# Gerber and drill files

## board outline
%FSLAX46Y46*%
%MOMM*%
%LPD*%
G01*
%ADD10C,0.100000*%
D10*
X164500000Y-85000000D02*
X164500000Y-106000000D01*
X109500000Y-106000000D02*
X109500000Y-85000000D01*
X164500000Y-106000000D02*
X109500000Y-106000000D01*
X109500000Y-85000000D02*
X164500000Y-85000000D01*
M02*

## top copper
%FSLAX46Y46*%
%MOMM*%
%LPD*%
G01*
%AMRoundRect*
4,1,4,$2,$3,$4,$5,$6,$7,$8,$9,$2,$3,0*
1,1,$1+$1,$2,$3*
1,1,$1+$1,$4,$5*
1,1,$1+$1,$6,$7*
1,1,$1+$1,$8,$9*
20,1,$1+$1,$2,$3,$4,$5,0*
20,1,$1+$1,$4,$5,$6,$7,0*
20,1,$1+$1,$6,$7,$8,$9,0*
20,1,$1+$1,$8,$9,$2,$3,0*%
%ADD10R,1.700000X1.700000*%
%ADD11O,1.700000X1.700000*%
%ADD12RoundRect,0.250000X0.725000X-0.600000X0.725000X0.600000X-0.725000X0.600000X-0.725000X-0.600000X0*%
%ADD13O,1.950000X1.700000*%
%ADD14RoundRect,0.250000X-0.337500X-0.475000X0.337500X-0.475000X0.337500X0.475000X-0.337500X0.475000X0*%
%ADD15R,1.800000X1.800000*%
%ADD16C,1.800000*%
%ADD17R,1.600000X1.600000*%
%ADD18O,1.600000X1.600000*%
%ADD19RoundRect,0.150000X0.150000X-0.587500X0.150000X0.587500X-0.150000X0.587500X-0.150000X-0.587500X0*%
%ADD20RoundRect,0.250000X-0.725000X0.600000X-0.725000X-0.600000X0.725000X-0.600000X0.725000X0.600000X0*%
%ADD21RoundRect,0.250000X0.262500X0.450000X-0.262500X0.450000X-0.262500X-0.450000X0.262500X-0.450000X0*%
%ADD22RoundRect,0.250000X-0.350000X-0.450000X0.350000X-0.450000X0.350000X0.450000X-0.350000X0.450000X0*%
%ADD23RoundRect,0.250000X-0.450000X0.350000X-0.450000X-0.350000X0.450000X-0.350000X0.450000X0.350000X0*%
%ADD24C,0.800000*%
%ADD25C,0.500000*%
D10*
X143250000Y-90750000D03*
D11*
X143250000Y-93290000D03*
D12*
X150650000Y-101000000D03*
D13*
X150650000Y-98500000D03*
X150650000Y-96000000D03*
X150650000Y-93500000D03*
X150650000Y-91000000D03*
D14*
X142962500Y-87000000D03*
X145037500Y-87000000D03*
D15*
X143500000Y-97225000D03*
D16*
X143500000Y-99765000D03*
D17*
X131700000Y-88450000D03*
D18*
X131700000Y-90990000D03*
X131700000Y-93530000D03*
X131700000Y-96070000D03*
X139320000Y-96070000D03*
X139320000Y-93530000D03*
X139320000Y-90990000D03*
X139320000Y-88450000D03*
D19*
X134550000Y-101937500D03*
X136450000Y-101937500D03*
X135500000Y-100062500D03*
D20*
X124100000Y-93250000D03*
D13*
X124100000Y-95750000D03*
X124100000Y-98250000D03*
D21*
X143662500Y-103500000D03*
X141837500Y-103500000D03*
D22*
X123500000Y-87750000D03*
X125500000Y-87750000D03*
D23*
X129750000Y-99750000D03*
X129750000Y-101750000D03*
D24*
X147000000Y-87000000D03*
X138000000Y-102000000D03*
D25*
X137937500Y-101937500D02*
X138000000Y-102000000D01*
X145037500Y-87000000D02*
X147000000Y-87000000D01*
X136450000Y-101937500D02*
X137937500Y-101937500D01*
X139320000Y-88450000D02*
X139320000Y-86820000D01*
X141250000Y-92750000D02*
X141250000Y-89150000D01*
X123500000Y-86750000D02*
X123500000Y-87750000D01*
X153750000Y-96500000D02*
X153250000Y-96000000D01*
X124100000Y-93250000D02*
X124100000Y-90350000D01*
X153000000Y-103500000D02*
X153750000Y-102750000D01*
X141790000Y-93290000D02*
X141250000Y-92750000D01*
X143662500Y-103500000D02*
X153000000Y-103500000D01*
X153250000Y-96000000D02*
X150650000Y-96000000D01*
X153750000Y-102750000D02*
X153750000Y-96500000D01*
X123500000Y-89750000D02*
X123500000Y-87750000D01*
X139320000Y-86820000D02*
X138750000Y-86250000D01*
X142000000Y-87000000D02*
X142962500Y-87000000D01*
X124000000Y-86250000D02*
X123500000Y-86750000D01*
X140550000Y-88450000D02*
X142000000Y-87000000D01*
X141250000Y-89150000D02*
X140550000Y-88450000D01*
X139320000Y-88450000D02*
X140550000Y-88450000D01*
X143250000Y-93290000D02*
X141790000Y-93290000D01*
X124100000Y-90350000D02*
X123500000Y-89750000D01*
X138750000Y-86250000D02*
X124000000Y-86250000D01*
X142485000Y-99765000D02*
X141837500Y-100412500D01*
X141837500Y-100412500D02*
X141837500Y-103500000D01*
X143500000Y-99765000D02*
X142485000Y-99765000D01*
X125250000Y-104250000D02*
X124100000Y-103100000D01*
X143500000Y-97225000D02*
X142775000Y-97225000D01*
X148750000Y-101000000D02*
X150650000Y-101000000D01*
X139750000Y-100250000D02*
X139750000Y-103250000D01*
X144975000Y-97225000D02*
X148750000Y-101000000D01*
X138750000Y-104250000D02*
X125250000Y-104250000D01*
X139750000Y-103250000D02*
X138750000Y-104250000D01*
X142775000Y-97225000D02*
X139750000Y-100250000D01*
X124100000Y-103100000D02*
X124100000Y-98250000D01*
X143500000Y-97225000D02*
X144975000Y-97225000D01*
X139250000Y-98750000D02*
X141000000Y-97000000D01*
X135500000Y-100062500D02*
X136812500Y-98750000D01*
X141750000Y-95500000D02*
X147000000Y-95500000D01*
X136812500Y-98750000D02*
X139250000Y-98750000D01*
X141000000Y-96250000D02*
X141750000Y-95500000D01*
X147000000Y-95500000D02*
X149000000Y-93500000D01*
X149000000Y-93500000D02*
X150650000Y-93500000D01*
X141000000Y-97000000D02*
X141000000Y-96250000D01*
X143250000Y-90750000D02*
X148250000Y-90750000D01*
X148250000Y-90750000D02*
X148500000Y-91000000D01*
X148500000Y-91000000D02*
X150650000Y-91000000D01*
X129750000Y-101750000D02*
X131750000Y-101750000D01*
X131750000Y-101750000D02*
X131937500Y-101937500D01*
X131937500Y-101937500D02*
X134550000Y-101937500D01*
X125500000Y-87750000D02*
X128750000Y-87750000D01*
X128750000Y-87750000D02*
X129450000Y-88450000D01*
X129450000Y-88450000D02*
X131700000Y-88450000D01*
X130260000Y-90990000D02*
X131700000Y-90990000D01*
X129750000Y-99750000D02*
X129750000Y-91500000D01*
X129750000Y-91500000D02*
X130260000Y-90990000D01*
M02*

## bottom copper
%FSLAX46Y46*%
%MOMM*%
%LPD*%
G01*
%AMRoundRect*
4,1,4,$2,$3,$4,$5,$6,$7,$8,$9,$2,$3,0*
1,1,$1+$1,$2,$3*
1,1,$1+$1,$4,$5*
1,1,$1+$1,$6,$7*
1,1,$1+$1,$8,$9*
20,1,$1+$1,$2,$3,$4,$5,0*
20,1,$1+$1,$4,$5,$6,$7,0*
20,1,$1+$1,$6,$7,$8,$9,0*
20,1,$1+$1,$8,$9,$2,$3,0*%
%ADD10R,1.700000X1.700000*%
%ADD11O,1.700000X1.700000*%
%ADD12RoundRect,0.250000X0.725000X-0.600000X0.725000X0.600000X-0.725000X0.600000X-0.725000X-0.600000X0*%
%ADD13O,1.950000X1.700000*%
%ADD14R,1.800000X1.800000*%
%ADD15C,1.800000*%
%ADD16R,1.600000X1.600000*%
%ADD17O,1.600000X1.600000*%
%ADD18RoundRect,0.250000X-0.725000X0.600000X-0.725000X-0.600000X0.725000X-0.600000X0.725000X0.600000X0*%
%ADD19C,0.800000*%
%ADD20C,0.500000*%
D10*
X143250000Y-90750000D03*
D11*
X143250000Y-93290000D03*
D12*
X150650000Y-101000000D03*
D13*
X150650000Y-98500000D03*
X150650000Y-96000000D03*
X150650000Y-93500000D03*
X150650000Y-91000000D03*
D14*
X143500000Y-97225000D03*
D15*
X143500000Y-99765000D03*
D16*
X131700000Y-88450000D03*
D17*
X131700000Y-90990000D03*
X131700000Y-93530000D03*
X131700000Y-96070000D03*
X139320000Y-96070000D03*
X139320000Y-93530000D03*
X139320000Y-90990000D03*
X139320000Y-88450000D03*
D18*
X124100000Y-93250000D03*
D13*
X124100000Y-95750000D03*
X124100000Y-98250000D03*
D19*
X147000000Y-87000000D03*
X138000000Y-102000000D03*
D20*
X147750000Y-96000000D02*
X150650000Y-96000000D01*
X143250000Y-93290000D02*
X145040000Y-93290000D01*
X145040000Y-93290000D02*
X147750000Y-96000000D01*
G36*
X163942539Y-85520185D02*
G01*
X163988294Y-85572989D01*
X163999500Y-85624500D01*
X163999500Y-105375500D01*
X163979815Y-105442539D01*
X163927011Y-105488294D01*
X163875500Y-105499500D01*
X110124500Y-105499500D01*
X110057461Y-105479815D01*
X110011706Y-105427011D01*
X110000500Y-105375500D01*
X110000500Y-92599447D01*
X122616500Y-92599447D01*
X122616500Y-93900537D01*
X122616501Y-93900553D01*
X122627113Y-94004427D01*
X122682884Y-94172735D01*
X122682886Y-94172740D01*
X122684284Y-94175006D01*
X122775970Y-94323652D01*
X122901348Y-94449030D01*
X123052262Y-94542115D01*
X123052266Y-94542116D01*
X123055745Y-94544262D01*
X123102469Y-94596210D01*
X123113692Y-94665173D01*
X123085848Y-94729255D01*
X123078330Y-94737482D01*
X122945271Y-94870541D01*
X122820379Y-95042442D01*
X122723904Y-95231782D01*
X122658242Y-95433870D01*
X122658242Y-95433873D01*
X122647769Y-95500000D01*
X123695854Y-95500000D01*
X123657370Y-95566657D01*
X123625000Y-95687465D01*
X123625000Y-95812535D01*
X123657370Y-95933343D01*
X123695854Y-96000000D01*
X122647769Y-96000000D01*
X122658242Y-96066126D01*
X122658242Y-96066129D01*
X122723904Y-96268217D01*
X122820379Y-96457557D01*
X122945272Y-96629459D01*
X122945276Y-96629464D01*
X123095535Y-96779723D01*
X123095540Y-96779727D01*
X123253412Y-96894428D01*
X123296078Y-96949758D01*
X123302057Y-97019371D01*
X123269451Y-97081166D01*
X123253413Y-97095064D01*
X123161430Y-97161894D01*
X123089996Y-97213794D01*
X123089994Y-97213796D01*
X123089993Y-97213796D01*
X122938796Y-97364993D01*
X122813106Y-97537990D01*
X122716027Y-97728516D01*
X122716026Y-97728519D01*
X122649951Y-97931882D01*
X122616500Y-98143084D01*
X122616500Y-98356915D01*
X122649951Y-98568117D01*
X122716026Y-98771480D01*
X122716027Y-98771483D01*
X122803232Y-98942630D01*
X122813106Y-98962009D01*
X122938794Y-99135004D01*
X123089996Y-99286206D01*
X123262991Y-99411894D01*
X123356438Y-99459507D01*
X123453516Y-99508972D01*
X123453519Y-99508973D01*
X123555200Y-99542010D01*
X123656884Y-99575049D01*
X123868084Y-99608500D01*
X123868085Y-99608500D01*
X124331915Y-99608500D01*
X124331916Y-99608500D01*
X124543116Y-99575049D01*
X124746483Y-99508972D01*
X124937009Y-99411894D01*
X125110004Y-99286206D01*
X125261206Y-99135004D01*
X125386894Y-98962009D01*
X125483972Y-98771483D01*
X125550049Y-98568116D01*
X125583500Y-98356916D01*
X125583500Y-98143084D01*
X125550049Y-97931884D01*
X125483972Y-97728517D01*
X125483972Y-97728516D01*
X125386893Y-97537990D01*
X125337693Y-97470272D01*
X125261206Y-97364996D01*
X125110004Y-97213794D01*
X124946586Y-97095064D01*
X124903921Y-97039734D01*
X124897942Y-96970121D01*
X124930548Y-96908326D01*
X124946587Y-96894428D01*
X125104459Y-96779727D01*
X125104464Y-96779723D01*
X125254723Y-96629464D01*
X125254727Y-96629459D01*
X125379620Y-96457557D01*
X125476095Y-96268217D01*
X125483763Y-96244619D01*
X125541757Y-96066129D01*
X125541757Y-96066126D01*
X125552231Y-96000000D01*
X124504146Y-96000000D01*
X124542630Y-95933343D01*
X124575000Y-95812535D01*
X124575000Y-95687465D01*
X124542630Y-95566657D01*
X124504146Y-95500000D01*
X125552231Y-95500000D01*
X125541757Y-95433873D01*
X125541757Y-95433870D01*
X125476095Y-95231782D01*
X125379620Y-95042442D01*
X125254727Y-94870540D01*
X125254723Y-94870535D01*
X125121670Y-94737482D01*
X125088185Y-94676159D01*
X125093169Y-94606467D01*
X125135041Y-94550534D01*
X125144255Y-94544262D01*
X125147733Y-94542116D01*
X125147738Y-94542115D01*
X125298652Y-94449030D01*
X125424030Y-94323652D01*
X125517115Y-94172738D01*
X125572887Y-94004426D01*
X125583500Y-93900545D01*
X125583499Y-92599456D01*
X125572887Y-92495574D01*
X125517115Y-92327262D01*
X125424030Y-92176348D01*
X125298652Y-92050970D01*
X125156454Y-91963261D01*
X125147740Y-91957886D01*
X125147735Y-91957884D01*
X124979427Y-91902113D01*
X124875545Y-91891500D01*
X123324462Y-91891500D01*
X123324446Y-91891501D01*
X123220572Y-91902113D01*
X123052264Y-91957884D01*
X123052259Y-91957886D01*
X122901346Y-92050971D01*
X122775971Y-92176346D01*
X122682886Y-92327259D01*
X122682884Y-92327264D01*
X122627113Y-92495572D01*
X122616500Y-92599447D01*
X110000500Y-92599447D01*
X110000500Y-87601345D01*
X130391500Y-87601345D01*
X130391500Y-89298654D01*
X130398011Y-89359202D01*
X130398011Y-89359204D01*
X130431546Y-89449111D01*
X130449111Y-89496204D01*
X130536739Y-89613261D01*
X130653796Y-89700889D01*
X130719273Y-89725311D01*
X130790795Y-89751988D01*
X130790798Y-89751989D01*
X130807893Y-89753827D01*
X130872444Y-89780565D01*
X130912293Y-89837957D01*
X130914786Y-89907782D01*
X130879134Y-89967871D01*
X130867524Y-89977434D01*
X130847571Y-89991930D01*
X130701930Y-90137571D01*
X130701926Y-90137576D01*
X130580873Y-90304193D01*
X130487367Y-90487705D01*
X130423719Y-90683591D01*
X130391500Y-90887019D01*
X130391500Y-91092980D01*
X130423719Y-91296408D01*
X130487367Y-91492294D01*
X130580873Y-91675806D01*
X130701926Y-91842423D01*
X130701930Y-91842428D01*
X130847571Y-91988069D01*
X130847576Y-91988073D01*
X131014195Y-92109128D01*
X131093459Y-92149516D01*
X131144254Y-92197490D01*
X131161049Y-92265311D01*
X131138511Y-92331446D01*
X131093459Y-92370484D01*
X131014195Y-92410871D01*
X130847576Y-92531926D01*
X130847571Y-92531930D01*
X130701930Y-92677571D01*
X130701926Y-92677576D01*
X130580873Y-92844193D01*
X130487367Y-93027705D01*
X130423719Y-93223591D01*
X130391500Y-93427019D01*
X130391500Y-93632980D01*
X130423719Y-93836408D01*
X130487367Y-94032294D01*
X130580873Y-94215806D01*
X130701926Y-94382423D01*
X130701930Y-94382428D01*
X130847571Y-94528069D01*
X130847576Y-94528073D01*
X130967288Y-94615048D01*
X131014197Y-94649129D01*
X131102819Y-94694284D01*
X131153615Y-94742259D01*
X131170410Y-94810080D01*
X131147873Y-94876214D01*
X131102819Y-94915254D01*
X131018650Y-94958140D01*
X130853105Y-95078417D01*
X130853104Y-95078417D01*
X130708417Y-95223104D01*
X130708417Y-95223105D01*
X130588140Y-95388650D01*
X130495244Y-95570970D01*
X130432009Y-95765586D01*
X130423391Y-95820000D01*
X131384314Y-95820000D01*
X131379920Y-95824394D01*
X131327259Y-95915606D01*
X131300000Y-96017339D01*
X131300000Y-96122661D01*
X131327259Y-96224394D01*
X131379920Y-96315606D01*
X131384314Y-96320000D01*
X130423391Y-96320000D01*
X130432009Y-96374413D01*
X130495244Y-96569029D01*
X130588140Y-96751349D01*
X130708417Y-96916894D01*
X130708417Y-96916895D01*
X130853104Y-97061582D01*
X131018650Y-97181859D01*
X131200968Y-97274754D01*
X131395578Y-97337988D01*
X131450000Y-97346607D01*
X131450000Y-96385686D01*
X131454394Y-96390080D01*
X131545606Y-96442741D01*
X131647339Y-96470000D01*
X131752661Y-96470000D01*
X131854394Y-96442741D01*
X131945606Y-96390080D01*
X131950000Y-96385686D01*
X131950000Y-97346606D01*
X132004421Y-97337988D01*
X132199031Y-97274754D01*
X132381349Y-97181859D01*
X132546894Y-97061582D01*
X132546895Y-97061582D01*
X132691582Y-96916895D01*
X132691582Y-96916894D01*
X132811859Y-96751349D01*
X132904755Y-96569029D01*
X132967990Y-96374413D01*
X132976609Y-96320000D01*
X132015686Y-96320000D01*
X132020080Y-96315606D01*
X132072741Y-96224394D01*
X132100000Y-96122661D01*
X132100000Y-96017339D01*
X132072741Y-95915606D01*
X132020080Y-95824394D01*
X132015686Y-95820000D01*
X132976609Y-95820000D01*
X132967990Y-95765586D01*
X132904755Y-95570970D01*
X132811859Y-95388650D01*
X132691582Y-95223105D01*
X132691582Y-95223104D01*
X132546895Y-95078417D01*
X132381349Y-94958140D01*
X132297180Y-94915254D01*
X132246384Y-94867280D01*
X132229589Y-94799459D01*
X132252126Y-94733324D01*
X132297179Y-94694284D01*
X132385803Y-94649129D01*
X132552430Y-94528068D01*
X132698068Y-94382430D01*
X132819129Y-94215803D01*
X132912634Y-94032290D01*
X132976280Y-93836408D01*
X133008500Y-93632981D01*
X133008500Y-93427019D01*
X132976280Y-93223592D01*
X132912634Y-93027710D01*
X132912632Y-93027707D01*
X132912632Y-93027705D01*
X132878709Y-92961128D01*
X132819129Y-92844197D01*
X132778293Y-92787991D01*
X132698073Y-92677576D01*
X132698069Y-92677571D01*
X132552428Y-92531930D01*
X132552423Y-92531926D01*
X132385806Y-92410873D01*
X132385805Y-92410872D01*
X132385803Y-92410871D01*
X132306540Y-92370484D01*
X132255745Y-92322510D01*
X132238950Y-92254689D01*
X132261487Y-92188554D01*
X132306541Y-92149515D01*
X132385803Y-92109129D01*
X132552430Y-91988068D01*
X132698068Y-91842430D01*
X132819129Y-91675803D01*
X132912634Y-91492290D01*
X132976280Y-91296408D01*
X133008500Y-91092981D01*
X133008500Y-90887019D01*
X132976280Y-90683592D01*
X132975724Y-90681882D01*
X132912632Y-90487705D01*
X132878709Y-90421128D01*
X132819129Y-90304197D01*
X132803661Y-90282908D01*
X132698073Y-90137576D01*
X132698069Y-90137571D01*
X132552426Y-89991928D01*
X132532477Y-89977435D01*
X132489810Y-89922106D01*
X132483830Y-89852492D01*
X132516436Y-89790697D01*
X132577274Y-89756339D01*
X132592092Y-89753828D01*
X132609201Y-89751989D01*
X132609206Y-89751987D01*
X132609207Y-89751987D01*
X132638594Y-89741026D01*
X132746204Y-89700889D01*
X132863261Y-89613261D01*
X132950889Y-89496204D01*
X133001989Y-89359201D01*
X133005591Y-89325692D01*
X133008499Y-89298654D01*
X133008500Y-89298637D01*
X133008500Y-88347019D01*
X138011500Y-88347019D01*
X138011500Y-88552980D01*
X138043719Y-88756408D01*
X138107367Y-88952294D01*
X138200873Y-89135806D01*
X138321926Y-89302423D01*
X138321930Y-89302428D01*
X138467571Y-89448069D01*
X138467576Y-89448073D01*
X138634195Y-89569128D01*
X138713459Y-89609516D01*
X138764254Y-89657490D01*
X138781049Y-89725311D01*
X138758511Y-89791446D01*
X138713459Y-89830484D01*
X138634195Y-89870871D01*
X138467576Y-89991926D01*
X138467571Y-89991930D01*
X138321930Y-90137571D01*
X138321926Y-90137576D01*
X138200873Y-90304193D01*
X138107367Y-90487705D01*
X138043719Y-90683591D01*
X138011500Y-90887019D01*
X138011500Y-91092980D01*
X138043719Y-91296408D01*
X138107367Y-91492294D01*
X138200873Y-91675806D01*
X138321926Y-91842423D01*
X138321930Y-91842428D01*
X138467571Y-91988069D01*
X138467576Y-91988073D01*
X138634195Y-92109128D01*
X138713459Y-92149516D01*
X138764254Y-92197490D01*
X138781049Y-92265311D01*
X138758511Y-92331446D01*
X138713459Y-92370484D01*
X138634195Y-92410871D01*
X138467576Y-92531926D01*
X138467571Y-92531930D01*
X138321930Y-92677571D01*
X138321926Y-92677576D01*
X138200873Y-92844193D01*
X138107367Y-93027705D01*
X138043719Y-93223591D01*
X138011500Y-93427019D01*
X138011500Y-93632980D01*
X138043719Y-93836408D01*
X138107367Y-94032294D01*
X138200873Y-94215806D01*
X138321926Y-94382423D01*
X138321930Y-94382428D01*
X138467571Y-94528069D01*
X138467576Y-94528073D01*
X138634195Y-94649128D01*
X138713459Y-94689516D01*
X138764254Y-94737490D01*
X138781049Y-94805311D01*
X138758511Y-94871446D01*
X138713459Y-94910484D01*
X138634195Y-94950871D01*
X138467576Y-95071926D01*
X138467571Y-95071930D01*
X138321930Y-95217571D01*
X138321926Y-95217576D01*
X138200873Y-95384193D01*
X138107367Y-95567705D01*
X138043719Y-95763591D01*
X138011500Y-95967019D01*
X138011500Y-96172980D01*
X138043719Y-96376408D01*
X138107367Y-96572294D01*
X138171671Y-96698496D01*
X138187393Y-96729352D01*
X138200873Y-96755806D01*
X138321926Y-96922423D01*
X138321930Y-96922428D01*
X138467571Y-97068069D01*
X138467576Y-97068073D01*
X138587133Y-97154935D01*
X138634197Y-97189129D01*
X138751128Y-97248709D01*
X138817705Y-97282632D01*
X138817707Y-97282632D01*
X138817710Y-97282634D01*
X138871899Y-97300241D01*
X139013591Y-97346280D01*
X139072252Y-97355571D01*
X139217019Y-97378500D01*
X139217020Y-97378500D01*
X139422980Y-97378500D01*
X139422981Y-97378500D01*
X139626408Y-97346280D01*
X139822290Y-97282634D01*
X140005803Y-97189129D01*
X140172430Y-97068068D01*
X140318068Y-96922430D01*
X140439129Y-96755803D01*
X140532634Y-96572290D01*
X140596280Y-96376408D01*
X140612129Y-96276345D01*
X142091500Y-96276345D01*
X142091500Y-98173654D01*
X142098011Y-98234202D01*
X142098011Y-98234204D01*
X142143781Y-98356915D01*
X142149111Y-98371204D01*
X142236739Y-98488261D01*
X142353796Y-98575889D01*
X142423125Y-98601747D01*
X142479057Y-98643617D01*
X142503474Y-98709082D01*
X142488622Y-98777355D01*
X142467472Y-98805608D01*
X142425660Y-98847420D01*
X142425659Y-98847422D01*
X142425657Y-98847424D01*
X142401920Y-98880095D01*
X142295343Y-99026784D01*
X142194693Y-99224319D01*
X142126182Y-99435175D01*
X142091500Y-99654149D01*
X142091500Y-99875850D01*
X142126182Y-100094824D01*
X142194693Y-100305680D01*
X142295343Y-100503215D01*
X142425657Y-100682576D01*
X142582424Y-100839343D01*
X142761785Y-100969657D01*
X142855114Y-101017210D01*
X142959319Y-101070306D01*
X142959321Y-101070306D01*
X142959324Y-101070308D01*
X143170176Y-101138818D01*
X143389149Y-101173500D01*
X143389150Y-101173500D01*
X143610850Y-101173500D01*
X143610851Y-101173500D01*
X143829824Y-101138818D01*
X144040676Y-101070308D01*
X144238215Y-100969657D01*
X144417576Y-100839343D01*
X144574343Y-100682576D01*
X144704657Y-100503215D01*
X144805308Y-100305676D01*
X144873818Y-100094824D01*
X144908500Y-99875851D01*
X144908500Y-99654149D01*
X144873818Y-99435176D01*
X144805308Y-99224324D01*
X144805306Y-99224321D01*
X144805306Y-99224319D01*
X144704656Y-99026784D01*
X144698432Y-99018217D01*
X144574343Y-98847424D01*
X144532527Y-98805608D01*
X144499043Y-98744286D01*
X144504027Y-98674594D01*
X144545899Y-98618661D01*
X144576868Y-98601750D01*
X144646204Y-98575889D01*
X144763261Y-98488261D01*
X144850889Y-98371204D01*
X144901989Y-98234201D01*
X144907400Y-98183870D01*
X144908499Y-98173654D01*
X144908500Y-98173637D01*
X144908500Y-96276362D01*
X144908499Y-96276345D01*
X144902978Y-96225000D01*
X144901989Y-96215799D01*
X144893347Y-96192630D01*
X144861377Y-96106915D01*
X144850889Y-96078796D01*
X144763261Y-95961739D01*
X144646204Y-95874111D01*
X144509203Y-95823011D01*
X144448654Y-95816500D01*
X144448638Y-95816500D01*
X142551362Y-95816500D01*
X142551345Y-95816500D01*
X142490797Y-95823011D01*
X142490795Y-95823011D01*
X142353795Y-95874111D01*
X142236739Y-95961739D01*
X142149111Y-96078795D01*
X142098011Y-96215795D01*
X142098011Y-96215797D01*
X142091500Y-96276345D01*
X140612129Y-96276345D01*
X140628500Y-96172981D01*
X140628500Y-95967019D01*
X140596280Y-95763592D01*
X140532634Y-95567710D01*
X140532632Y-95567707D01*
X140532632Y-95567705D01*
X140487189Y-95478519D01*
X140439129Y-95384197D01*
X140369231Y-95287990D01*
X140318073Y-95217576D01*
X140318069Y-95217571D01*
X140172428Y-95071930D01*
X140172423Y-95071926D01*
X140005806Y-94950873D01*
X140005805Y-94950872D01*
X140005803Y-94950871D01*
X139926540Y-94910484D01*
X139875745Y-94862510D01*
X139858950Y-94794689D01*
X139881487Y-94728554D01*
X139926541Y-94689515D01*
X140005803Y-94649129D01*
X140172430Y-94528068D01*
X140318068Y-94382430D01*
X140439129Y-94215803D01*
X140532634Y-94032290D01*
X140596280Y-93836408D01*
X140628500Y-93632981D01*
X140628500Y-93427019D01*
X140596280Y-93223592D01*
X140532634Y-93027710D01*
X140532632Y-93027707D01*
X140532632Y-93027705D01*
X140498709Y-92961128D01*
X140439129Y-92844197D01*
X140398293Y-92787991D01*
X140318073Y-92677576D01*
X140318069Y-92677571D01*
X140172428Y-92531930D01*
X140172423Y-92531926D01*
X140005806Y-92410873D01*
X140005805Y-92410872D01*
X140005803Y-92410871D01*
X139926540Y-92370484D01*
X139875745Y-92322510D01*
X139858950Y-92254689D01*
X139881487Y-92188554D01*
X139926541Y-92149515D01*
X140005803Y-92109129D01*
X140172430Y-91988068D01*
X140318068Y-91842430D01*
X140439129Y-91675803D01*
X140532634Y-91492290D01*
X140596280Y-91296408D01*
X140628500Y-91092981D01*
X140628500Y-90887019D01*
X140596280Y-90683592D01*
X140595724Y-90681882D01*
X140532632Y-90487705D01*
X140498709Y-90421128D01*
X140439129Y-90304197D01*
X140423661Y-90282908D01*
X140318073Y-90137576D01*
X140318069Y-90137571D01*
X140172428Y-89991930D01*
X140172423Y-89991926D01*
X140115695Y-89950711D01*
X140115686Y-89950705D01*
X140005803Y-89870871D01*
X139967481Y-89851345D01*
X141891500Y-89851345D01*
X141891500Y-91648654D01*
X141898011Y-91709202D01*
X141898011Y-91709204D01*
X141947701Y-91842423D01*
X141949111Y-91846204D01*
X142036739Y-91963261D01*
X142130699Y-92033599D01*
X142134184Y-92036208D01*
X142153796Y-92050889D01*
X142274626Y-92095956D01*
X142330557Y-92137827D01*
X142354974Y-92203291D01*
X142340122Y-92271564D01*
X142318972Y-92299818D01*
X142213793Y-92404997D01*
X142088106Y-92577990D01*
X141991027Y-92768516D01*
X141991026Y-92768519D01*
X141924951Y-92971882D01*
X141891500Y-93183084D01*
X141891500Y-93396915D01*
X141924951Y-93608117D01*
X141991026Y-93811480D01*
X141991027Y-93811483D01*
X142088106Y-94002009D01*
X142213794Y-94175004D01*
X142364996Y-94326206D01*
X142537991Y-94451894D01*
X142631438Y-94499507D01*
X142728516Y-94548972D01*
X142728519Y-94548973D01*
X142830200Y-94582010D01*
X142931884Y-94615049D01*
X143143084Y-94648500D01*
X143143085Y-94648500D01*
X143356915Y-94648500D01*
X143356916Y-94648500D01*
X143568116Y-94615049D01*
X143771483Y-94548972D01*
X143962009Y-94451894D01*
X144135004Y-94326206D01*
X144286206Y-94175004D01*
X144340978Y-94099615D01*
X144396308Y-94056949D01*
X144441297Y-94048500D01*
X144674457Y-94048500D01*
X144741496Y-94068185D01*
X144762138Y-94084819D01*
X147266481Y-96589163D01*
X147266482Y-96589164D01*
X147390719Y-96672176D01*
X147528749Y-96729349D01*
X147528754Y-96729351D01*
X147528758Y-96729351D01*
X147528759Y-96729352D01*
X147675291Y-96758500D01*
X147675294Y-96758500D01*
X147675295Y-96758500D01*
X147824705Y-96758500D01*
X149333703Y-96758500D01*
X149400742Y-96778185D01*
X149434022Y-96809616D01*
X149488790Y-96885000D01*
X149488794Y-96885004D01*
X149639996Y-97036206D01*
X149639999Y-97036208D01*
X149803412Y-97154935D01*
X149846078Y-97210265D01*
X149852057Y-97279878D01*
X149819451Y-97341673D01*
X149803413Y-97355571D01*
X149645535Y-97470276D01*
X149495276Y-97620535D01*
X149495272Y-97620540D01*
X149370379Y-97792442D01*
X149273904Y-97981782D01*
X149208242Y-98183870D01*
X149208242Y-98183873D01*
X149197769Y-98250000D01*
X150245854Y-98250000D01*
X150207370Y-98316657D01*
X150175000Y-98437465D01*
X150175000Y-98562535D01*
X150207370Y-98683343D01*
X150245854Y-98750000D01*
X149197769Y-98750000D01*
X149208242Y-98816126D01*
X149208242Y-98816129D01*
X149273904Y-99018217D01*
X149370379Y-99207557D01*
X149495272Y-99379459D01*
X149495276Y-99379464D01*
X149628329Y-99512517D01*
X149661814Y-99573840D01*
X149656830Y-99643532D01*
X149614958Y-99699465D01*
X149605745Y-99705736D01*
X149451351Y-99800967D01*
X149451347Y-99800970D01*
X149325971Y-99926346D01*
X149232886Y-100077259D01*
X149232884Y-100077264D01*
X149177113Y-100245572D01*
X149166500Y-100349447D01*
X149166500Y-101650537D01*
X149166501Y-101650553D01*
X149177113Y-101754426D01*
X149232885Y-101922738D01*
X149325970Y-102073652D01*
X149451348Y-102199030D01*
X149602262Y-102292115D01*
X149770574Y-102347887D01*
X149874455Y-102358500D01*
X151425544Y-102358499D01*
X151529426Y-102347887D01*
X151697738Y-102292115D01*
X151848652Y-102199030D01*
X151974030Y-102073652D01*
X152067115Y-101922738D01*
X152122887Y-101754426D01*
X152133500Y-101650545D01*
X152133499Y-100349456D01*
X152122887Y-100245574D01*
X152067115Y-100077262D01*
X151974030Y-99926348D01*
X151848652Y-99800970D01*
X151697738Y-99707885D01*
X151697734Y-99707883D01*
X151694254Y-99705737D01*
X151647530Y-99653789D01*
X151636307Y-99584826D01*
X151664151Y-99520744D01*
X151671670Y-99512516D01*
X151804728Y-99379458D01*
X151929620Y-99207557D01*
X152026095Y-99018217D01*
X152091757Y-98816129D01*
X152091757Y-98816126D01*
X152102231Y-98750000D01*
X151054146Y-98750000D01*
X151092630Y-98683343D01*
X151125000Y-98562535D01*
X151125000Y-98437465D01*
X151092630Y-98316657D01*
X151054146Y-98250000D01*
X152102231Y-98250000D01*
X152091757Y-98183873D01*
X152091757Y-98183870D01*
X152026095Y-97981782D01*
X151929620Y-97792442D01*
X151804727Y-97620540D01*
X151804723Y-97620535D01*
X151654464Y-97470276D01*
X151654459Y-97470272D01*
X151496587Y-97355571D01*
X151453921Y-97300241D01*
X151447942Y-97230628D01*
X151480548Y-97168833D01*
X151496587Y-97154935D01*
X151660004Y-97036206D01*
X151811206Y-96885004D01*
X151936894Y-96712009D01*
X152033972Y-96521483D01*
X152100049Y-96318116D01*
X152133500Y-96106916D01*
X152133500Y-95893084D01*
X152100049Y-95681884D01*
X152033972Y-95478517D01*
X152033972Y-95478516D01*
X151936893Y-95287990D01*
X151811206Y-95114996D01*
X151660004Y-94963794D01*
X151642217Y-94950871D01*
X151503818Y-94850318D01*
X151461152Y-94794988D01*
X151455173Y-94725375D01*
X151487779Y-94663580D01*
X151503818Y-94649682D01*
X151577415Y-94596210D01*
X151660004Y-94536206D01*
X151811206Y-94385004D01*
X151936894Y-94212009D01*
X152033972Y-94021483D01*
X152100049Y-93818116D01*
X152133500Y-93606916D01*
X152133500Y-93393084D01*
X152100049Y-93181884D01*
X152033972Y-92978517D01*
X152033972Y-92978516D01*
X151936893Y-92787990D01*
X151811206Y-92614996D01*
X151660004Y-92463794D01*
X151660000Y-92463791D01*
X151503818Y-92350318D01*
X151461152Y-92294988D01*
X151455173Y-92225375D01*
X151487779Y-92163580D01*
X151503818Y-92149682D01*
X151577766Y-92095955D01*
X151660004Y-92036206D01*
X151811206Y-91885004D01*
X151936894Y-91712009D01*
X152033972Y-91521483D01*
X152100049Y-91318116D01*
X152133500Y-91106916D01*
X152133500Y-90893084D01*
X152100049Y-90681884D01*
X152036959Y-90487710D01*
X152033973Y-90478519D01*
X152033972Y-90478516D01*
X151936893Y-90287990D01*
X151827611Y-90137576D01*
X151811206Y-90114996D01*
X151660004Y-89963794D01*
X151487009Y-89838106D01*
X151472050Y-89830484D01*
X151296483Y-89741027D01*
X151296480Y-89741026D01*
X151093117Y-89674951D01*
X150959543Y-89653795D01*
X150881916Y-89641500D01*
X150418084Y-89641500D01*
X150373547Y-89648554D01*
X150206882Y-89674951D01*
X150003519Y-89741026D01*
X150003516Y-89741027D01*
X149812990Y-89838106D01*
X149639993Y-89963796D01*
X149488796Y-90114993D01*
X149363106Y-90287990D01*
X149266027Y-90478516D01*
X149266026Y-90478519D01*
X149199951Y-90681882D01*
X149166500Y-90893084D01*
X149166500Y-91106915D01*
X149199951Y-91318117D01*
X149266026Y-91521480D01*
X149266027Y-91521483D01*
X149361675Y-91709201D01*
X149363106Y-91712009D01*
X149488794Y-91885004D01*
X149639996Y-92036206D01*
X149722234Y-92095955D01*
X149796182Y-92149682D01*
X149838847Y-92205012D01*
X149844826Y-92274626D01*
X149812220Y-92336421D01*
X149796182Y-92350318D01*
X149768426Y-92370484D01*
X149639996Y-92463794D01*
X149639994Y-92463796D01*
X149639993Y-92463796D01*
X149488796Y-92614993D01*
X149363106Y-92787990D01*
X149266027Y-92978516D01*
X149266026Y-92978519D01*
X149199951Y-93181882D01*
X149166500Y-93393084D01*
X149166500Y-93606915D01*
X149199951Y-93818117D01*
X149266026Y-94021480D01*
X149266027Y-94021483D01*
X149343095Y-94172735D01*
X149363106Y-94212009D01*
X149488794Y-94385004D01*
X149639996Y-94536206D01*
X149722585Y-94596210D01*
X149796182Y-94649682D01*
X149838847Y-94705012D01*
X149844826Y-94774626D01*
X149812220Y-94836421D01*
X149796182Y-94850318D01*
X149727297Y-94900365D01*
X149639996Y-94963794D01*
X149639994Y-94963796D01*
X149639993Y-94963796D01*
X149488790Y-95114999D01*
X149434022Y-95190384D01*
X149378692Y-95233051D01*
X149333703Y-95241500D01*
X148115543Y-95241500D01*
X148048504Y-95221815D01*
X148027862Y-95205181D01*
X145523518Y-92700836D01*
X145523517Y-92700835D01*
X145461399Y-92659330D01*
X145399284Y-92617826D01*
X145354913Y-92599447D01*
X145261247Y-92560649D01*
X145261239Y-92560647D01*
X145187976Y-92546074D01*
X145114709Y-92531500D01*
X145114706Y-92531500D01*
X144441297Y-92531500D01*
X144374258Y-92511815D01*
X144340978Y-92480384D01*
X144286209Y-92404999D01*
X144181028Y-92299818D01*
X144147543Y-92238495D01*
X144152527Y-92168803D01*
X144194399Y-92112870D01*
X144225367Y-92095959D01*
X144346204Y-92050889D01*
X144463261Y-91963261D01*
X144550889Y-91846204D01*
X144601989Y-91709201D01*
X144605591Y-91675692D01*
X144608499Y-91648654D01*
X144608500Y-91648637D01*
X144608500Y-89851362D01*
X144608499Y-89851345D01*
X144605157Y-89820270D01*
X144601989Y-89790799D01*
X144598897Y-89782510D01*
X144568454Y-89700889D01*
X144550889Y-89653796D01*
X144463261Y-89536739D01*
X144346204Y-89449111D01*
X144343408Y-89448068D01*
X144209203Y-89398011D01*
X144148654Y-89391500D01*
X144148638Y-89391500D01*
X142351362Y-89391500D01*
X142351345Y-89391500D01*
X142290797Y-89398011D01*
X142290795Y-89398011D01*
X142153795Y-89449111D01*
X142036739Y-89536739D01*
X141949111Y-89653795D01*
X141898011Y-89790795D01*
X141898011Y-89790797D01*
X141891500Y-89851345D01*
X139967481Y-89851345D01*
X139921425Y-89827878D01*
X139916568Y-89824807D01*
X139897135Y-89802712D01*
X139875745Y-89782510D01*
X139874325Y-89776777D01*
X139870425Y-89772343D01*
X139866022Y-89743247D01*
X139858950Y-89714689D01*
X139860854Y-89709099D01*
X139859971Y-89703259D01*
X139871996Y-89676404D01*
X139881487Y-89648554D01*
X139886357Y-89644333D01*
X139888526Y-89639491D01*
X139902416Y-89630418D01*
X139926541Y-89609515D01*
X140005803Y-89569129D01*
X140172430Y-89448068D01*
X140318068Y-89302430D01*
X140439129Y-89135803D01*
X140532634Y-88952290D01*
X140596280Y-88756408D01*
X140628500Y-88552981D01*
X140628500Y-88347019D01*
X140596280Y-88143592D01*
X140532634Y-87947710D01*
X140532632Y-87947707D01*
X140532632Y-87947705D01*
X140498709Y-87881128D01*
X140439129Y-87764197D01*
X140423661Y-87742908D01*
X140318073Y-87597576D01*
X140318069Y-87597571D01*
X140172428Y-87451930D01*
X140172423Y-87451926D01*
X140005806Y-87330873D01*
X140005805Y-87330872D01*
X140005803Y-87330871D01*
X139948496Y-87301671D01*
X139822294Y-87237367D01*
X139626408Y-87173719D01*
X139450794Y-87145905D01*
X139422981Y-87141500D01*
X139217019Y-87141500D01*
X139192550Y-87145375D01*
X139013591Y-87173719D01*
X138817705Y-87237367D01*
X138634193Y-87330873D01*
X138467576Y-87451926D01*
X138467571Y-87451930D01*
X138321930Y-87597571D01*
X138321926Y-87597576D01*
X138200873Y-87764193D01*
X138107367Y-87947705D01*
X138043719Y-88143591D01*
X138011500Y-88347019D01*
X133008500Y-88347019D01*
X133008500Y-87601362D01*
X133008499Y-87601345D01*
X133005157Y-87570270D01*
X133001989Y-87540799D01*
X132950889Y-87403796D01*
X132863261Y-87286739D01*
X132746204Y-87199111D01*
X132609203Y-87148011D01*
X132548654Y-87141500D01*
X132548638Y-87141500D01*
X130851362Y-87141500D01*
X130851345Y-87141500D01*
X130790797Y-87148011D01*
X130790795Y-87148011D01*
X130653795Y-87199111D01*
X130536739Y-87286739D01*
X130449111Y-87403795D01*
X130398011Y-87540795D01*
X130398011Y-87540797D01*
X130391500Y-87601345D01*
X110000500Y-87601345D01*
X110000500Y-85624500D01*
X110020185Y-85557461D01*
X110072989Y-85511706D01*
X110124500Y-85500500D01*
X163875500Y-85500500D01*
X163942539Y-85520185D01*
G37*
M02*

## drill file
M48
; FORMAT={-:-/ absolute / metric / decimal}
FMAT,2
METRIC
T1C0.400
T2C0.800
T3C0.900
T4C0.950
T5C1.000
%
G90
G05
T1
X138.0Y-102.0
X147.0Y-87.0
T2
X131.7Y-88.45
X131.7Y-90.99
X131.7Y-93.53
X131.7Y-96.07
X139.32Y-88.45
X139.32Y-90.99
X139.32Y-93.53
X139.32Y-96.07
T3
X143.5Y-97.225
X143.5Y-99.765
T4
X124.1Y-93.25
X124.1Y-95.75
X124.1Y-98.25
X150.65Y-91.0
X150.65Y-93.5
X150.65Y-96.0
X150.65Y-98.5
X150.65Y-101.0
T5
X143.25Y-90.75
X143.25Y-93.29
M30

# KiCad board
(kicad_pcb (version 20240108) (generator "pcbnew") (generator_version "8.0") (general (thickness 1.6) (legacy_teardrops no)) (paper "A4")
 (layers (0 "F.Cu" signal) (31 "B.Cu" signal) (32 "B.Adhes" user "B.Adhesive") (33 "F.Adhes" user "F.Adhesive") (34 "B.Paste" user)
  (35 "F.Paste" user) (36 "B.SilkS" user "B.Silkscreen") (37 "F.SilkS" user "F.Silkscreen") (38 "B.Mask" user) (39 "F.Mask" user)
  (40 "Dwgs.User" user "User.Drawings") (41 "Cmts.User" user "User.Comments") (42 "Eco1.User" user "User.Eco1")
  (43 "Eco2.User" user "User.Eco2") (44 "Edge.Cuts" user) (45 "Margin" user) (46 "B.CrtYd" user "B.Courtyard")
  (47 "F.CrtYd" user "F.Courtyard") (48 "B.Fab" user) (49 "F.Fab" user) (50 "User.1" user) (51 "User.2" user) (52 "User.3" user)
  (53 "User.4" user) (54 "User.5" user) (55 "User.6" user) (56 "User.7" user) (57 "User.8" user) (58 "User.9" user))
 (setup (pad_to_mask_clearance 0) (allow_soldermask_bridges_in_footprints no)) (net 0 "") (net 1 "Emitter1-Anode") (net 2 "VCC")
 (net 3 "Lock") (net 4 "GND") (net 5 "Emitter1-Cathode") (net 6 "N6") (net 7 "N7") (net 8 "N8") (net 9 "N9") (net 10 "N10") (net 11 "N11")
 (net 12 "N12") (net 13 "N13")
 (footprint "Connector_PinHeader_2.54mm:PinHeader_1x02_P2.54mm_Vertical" (layer "F.Cu") (at 143.25 90.75)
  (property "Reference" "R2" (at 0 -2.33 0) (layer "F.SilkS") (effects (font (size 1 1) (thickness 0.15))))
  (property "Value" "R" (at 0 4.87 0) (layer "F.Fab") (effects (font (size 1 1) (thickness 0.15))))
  (pad "1" thru_hole rect (at 0 0) (size 1.7 1.7) (drill 1) (layers "*.Cu" "*.Mask") (remove_unused_layers no) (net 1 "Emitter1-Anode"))
  (pad "2" thru_hole oval (at 0 2.54) (size 1.7 1.7) (drill 1) (layers "*.Cu" "*.Mask") (remove_unused_layers no) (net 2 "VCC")))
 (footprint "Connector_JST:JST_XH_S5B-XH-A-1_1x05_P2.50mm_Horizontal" (layer "F.Cu") (at 150.65 101 90)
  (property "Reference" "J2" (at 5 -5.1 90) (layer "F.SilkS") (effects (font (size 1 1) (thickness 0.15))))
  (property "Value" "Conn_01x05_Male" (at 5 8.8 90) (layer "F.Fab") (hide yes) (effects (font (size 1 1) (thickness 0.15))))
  (pad "1" thru_hole roundrect (at 0 0 90) (size 1.7 1.95) (drill 0.95) (layers "*.Cu" "*.Mask") (remove_unused_layers no)
   (roundrect_rratio 0.147059) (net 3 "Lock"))
  (pad "2" thru_hole oval (at 2.5 0 90) (size 1.7 1.95) (drill 0.95) (layers "*.Cu" "*.Mask") (remove_unused_layers no) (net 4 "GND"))
  (pad "3" thru_hole oval (at 5 0 90) (size 1.7 1.95) (drill 0.95) (layers "*.Cu" "*.Mask") (remove_unused_layers no) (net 2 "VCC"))
  (pad "4" thru_hole oval (at 7.5 0 90) (size 1.7 1.95) (drill 0.95) (layers "*.Cu" "*.Mask") (remove_unused_layers no)
   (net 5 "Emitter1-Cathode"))
  (pad "5" thru_hole oval (at 10 0 90) (size 1.7 1.95) (drill 0.95) (layers "*.Cu" "*.Mask") (remove_unused_layers no)
   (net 1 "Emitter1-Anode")))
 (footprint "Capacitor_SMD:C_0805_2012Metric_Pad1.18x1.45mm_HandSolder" (layer "F.Cu") (at 144 87)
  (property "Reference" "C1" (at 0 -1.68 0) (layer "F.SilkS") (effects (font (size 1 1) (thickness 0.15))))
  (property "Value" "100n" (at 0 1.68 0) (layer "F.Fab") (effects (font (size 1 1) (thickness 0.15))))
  (pad "1" smd roundrect (at -1.0375 0) (size 1.175 1.45) (layers "F.Cu" "F.Paste" "F.Mask") (roundrect_rratio 0.212766) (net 2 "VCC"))
  (pad "2" smd roundrect (at 1.0375 0) (size 1.175 1.45) (layers "F.Cu" "F.Paste" "F.Mask") (roundrect_rratio 0.212766) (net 4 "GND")))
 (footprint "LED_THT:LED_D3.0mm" (layer "F.Cu") (at 143.5 97.225 -90)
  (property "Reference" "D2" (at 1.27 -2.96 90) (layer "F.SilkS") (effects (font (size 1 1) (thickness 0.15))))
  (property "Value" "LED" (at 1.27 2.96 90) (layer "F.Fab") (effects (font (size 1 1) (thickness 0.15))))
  (pad "1" thru_hole rect (at 0 0 270) (size 1.8 1.8) (drill 0.9) (layers "*.Cu" "*.Mask") (remove_unused_layers no) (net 3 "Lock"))
  (pad "2" thru_hole circle (at 2.54 0 270) (size 1.8 1.8) (drill 0.9) (layers "*.Cu" "*.Mask") (remove_unused_layers no) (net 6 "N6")))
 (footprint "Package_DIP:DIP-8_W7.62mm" (layer "F.Cu") (at 131.7 88.45)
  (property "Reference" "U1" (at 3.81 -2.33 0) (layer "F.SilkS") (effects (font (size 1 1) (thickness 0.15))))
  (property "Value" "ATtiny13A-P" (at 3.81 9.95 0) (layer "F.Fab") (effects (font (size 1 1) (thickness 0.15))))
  (pad "1" thru_hole rect (at 0 0) (size 1.6 1.6) (drill 0.8) (layers "*.Cu" "*.Mask") (remove_unused_layers no) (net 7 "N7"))
  (pad "2" thru_hole oval (at 0 2.54) (size 1.6 1.6) (drill 0.8) (layers "*.Cu" "*.Mask") (remove_unused_layers no) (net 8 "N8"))
  (pad "3" thru_hole oval (at 0 5.08) (size 1.6 1.6) (drill 0.8) (layers "*.Cu" "*.Mask") (remove_unused_layers no) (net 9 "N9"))
  (pad "4" thru_hole oval (at 0 7.62) (size 1.6 1.6) (drill 0.8) (layers "*.Cu" "*.Mask") (remove_unused_layers no) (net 4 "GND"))
  (pad "5" thru_hole oval (at 7.62 7.62) (size 1.6 1.6) (drill 0.8) (layers "*.Cu" "*.Mask") (remove_unused_layers no) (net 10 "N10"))
  (pad "6" thru_hole oval (at 7.62 5.08) (size 1.6 1.6) (drill 0.8) (layers "*.Cu" "*.Mask") (remove_unused_layers no) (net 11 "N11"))
  (pad "7" thru_hole oval (at 7.62 2.54) (size 1.6 1.6) (drill 0.8) (layers "*.Cu" "*.Mask") (remove_unused_layers no) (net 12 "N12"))
  (pad "8" thru_hole oval (at 7.62 0) (size 1.6 1.6) (drill 0.8) (layers "*.Cu" "*.Mask") (remove_unused_layers no) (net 2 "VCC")))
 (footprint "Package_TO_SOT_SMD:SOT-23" (layer "F.Cu") (at 135.5 101 90)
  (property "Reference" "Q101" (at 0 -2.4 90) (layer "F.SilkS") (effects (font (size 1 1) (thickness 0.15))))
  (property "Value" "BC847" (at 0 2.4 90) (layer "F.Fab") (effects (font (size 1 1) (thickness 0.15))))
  (pad "1" smd roundrect (at -0.9375 -0.95 90) (size 1.475 0.6) (layers "F.Cu" "F.Paste" "F.Mask") (roundrect_rratio 0.25) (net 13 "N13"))
  (pad "2" smd roundrect (at -0.9375 0.95 90) (size 1.475 0.6) (layers "F.Cu" "F.Paste" "F.Mask") (roundrect_rratio 0.25) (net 4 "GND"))
  (pad "3" smd roundrect (at 0.9375 0 90) (size 1.475 0.6) (layers "F.Cu" "F.Paste" "F.Mask") (roundrect_rratio 0.25)
   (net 5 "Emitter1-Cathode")))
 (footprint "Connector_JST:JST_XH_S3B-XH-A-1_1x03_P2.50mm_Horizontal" (layer "F.Cu") (at 124.1 93.25 -90)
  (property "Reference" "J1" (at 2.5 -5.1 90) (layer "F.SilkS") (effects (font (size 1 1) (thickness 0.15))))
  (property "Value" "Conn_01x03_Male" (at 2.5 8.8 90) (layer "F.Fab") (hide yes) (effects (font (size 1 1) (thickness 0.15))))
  (pad "1" thru_hole roundrect (at 0 0 270) (size 1.7 1.95) (drill 0.95) (layers "*.Cu" "*.Mask") (remove_unused_layers no)
   (roundrect_rratio 0.147059) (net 2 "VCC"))
  (pad "2" thru_hole oval (at 2.5 0 270) (size 1.7 1.95) (drill 0.95) (layers "*.Cu" "*.Mask") (remove_unused_layers no) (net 4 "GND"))
  (pad "3" thru_hole oval (at 5 0 270) (size 1.7 1.95) (drill 0.95) (layers "*.Cu" "*.Mask") (remove_unused_layers no) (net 3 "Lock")))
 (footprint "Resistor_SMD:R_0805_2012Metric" (layer "F.Cu") (at 142.75 103.5 180)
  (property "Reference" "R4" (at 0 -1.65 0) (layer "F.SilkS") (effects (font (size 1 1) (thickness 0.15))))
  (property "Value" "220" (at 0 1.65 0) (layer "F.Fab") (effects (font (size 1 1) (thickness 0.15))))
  (pad "1" smd roundrect (at -0.9125 0 180) (size 1.025 1.4) (layers "F.Cu" "F.Paste" "F.Mask") (roundrect_rratio 0.243902) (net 2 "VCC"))
  (pad "2" smd roundrect (at 0.9125 0 180) (size 1.025 1.4) (layers "F.Cu" "F.Paste" "F.Mask") (roundrect_rratio 0.243902) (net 6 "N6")))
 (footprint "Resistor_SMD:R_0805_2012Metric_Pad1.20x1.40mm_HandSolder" (layer "F.Cu") (at 124.5 87.75)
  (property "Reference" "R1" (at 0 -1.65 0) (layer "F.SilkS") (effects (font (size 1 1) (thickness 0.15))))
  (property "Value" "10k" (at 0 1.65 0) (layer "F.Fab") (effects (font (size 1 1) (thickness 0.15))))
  (pad "1" smd roundrect (at -1 0) (size 1.2 1.4) (layers "F.Cu" "F.Paste" "F.Mask") (roundrect_rratio 0.208333) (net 2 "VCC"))
  (pad "2" smd roundrect (at 1 0) (size 1.2 1.4) (layers "F.Cu" "F.Paste" "F.Mask") (roundrect_rratio 0.208333) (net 7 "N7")))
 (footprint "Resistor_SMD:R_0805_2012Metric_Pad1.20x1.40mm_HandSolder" (layer "F.Cu") (at 129.75 100.75 -90)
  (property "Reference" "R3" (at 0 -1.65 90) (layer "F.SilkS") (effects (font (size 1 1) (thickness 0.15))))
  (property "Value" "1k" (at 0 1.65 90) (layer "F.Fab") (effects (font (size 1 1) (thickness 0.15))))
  (pad "1" smd roundrect (at -1 0 270) (size 1.2 1.4) (layers "F.Cu" "F.Paste" "F.Mask") (roundrect_rratio 0.208333) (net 8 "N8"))
  (pad "2" smd roundrect (at 1 0 270) (size 1.2 1.4) (layers "F.Cu" "F.Paste" "F.Mask") (roundrect_rratio 0.208333) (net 13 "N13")))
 (gr_line (start 164.5 85) (end 164.5 106) (stroke (width 0.1) (type solid)) (layer "Edge.Cuts"))
 (gr_line (start 109.5 106) (end 109.5 85) (stroke (width 0.1) (type solid)) (layer "Edge.Cuts"))
 (gr_line (start 164.5 106) (end 109.5 106) (stroke (width 0.1) (type solid)) (layer "Edge.Cuts"))
 (gr_line (start 109.5 85) (end 164.5 85) (stroke (width 0.1) (type solid)) (layer "Edge.Cuts"))
 (segment (start 137.9375 101.9375) (end 138 102) (width 0.5) (layer "F.Cu") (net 4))
 (segment (start 145.0375 87) (end 147 87) (width 0.5) (layer "F.Cu") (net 4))
 (segment (start 136.45 101.9375) (end 137.9375 101.9375) (width 0.5) (layer "F.Cu") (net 4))
 (via (at 147 87) (size 0.8) (drill 0.4) (layers "F.Cu" "B.Cu") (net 4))
 (via (at 138 102) (size 0.8) (drill 0.4) (layers "F.Cu" "B.Cu") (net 4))
 (segment (start 139.32 88.45) (end 139.32 86.82) (width 0.5) (layer "F.Cu") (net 2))
 (segment (start 141.25 92.75) (end 141.25 89.15) (width 0.5) (layer "F.Cu") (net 2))
 (segment (start 123.5 86.75) (end 123.5 87.75) (width 0.5) (layer "F.Cu") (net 2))
 (segment (start 153.75 96.5) (end 153.25 96) (width 0.5) (layer "F.Cu") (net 2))
 (segment (start 124.1 93.25) (end 124.1 90.35) (width 0.5) (layer "F.Cu") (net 2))
 (segment (start 153 103.5) (end 153.75 102.75) (width 0.5) (layer "F.Cu") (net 2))
 (segment (start 141.79 93.29) (end 141.25 92.75) (width 0.5) (layer "F.Cu") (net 2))
 (segment (start 143.6625 103.5) (end 153 103.5) (width 0.5) (layer "F.Cu") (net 2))
 (segment (start 153.25 96) (end 150.65 96) (width 0.5) (layer "F.Cu") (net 2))
 (segment (start 153.75 102.75) (end 153.75 96.5) (width 0.5) (layer "F.Cu") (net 2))
 (segment (start 123.5 89.75) (end 123.5 87.75) (width 0.5) (layer "F.Cu") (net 2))
 (segment (start 139.32 86.82) (end 138.75 86.25) (width 0.5) (layer "F.Cu") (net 2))
 (segment (start 142 87) (end 142.9625 87) (width 0.5) (layer "F.Cu") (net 2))
 (segment (start 124 86.25) (end 123.5 86.75) (width 0.5) (layer "F.Cu") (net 2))
 (segment (start 140.55 88.45) (end 142 87) (width 0.5) (layer "F.Cu") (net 2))
 (segment (start 141.25 89.15) (end 140.55 88.45) (width 0.5) (layer "F.Cu") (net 2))
 (segment (start 139.32 88.45) (end 140.55 88.45) (width 0.5) (layer "F.Cu") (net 2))
 (segment (start 143.25 93.29) (end 141.79 93.29) (width 0.5) (layer "F.Cu") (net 2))
 (segment (start 124.1 90.35) (end 123.5 89.75) (width 0.5) (layer "F.Cu") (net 2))
 (segment (start 138.75 86.25) (end 124 86.25) (width 0.5) (layer "F.Cu") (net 2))
 (segment (start 147.75 96) (end 150.65 96) (width 0.5) (layer "B.Cu") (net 2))
 (segment (start 143.25 93.29) (end 145.04 93.29) (width 0.5) (layer "B.Cu") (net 2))
 (segment (start 145.04 93.29) (end 147.75 96) (width 0.5) (layer "B.Cu") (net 2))
 (segment (start 142.485 99.765) (end 141.8375 100.4125) (width 0.5) (layer "F.Cu") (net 6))
 (segment (start 141.8375 100.4125) (end 141.8375 103.5) (width 0.5) (layer "F.Cu") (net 6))
 (segment (start 143.5 99.765) (end 142.485 99.765) (width 0.5) (layer "F.Cu") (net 6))
 (segment (start 125.25 104.25) (end 124.1 103.1) (width 0.5) (layer "F.Cu") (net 3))
 (segment (start 143.5 97.225) (end 142.775 97.225) (width 0.5) (layer "F.Cu") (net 3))
 (segment (start 148.75 101) (end 150.65 101) (width 0.5) (layer "F.Cu") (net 3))
 (segment (start 139.75 100.25) (end 139.75 103.25) (width 0.5) (layer "F.Cu") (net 3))
 (segment (start 144.975 97.225) (end 148.75 101) (width 0.5) (layer "F.Cu") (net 3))
 (segment (start 138.75 104.25) (end 125.25 104.25) (width 0.5) (layer "F.Cu") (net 3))
 (segment (start 139.75 103.25) (end 138.75 104.25) (width 0.5) (layer "F.Cu") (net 3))
 (segment (start 142.775 97.225) (end 139.75 100.25) (width 0.5) (layer "F.Cu") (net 3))
 (segment (start 124.1 103.1) (end 124.1 98.25) (width 0.5) (layer "F.Cu") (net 3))
 (segment (start 143.5 97.225) (end 144.975 97.225) (width 0.5) (layer "F.Cu") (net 3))
 (segment (start 139.25 98.75) (end 141 97) (width 0.5) (layer "F.Cu") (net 5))
 (segment (start 135.5 100.0625) (end 136.8125 98.75) (width 0.5) (layer "F.Cu") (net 5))
 (segment (start 141.75 95.5) (end 147 95.5) (width 0.5) (layer "F.Cu") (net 5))
 (segment (start 136.8125 98.75) (end 139.25 98.75) (width 0.5) (layer "F.Cu") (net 5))
 (segment (start 141 96.25) (end 141.75 95.5) (width 0.5) (layer "F.Cu") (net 5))
 (segment (start 147 95.5) (end 149 93.5) (width 0.5) (layer "F.Cu") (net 5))
 (segment (start 149 93.5) (end 150.65 93.5) (width 0.5) (layer "F.Cu") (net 5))
 (segment (start 141 97) (end 141 96.25) (width 0.5) (layer "F.Cu") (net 5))
 (segment (start 143.25 90.75) (end 148.25 90.75) (width 0.5) (layer "F.Cu") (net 1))
 (segment (start 148.25 90.75) (end 148.5 91) (width 0.5) (layer "F.Cu") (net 1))
 (segment (start 148.5 91) (end 150.65 91) (width 0.5) (layer "F.Cu") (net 1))
 (segment (start 129.75 101.75) (end 131.75 101.75) (width 0.5) (layer "F.Cu") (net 13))
 (segment (start 131.75 101.75) (end 131.9375 101.9375) (width 0.5) (layer "F.Cu") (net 13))
 (segment (start 131.9375 101.9375) (end 134.55 101.9375) (width 0.5) (layer "F.Cu") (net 13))
 (segment (start 125.5 87.75) (end 128.75 87.75) (width 0.5) (layer "F.Cu") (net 7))
 (segment (start 128.75 87.75) (end 129.45 88.45) (width 0.5) (layer "F.Cu") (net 7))
 (segment (start 129.45 88.45) (end 131.7 88.45) (width 0.5) (layer "F.Cu") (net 7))
 (segment (start 130.26 90.99) (end 131.7 90.99) (width 0.5) (layer "F.Cu") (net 8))
 (segment (start 129.75 99.75) (end 129.75 91.5) (width 0.5) (layer "F.Cu") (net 8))
 (segment (start 129.75 91.5) (end 130.26 90.99) (width 0.5) (layer "F.Cu") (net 8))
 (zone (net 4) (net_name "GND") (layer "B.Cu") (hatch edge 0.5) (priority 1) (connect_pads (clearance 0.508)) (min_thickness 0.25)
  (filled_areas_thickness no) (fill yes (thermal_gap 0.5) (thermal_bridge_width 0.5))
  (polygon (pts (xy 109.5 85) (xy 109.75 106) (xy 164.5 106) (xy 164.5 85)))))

